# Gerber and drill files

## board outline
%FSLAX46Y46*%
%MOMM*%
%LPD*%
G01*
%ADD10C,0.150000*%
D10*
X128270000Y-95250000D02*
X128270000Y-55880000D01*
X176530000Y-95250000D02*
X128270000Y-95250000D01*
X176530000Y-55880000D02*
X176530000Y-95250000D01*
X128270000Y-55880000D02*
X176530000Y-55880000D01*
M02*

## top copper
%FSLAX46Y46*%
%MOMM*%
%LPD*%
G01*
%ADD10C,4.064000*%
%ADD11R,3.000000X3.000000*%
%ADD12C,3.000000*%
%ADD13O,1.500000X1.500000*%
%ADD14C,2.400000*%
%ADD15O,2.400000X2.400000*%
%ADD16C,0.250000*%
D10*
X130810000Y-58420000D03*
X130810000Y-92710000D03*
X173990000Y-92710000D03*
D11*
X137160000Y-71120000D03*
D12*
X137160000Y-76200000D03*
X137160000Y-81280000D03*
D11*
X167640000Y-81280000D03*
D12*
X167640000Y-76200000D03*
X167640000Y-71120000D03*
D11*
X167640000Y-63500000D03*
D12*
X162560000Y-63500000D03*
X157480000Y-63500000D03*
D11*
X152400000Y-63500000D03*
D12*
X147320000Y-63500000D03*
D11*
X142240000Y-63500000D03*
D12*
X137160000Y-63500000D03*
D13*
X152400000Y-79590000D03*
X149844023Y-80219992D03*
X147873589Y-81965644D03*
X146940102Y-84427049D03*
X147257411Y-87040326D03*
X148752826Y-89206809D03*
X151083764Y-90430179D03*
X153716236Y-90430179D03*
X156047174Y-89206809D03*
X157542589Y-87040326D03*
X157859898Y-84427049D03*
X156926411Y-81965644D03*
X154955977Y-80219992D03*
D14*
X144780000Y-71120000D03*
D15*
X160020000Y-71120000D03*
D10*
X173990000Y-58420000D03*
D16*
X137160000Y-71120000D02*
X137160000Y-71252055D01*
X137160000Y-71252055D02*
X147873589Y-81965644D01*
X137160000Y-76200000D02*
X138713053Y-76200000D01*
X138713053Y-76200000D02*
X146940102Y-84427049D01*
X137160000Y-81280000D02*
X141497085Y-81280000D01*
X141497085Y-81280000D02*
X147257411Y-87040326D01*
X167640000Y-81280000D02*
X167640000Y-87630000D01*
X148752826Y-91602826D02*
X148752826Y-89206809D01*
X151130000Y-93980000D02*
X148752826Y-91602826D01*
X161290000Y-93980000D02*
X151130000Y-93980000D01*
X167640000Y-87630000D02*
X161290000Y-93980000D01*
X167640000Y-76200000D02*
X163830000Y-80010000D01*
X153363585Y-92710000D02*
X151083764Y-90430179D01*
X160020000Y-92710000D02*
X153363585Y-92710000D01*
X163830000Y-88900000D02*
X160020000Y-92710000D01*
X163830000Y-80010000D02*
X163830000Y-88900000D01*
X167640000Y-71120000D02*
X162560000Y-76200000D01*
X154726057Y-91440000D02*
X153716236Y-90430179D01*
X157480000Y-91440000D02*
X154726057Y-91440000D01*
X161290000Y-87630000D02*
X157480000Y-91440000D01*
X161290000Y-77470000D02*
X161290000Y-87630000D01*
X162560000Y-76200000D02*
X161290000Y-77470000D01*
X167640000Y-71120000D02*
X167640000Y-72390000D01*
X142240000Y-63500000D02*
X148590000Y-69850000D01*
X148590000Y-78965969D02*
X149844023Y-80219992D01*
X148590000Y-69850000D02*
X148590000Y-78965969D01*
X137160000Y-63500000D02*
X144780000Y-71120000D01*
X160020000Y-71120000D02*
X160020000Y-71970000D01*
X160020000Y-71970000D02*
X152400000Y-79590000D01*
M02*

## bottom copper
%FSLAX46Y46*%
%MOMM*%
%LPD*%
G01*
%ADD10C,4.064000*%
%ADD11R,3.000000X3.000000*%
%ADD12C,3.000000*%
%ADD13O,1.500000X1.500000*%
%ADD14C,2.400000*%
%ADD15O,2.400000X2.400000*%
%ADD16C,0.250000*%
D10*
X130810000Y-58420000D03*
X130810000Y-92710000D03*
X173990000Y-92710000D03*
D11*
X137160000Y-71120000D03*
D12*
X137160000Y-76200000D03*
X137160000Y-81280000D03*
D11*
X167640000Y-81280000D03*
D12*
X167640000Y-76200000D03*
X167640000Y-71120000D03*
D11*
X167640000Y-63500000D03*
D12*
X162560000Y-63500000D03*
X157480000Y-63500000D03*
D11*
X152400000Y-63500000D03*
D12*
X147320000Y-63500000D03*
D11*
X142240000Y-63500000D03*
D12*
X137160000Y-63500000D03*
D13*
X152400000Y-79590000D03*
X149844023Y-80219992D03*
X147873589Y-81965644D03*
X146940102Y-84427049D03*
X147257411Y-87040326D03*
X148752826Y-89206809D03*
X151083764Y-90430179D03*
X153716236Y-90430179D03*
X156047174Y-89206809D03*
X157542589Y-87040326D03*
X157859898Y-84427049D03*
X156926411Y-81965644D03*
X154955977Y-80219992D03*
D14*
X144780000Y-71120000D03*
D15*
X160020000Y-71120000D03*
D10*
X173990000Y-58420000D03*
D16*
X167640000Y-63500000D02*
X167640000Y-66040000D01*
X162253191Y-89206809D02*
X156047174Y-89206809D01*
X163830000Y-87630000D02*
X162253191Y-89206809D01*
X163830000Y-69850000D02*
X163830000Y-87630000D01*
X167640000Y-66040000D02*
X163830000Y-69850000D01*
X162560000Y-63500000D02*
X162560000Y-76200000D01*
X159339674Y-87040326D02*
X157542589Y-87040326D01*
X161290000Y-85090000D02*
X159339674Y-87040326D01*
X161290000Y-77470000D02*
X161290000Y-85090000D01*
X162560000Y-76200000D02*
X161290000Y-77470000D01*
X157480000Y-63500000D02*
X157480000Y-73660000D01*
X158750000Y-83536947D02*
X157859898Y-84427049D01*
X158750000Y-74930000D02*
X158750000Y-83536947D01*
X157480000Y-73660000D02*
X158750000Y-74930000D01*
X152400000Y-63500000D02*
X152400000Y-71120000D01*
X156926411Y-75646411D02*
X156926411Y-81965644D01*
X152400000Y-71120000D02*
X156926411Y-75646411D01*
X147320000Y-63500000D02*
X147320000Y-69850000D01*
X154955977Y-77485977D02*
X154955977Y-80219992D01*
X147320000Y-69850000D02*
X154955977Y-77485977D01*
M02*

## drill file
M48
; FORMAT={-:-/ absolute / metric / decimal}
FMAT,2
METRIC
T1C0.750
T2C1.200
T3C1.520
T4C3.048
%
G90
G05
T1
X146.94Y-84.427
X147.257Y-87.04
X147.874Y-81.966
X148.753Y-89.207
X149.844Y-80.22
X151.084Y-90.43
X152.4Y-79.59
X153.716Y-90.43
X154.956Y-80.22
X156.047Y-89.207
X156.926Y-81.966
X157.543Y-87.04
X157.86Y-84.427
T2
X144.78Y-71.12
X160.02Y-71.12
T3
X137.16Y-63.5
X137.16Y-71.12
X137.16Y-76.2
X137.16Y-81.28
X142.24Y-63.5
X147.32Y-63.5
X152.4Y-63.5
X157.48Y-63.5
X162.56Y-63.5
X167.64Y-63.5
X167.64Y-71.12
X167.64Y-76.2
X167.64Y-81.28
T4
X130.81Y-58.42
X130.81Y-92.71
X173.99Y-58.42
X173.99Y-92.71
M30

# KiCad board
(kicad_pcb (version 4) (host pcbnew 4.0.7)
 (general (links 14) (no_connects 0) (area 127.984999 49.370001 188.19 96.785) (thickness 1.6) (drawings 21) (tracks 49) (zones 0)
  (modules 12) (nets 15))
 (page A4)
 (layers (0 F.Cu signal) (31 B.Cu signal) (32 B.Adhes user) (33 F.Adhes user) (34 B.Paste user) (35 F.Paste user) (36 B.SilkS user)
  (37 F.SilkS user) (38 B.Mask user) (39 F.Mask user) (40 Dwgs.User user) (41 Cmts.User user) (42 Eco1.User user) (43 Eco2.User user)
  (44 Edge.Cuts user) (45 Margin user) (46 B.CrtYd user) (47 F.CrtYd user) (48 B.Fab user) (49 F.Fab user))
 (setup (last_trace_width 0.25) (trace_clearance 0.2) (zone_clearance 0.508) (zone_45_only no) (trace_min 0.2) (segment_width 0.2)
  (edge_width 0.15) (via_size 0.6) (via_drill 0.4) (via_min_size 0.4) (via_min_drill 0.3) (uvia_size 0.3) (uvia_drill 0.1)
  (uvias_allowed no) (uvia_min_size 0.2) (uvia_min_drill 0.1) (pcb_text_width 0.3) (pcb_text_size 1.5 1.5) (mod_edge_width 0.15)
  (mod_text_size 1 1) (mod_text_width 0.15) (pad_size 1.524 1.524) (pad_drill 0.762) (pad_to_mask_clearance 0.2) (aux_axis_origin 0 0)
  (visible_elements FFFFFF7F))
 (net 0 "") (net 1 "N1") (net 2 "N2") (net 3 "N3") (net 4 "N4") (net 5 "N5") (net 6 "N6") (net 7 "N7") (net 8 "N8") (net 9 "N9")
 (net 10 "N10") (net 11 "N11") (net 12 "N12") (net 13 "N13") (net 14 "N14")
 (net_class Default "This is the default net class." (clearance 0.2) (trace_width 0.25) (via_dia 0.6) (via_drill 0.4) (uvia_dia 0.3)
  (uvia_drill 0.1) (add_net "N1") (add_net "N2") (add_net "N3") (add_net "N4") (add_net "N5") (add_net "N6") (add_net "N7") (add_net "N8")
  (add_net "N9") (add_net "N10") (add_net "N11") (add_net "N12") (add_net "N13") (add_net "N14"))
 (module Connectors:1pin (layer F.Cu) (at 130.81 58.42)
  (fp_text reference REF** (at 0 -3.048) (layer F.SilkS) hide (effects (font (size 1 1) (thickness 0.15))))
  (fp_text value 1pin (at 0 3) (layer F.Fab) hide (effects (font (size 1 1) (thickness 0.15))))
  (pad 1 thru_hole circle (at 0 0) (size 4.064 4.064) (drill 3.048) (layers *.Cu *.Mask)))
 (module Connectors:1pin (layer F.Cu) (at 130.81 92.71)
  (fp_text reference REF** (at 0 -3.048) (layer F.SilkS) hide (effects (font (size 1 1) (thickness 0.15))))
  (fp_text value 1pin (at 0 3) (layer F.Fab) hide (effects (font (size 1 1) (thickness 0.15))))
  (pad 1 thru_hole circle (at 0 0) (size 4.064 4.064) (drill 3.048) (layers *.Cu *.Mask)))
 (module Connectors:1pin (layer F.Cu) (at 173.99 92.71)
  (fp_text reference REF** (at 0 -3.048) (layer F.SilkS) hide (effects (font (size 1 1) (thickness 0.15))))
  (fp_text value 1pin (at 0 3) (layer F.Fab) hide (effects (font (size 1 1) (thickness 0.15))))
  (pad 1 thru_hole circle (at 0 0) (size 4.064 4.064) (drill 3.048) (layers *.Cu *.Mask)))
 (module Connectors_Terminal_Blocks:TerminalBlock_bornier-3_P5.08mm (layer F.Cu) (at 137.16 71.12 270)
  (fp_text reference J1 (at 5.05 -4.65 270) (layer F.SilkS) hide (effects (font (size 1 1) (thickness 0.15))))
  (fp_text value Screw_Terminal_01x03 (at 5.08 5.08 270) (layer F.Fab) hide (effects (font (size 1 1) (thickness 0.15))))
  (pad 1 thru_hole rect (at 0 0 270) (size 3 3) (drill 1.52) (layers *.Cu *.Mask) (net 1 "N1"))
  (pad 2 thru_hole circle (at 5.08 0 270) (size 3 3) (drill 1.52) (layers *.Cu *.Mask) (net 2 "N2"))
  (pad 3 thru_hole circle (at 10.16 0 270) (size 3 3) (drill 1.52) (layers *.Cu *.Mask) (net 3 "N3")))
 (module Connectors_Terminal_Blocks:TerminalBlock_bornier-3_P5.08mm (layer F.Cu) (at 167.64 81.28 90)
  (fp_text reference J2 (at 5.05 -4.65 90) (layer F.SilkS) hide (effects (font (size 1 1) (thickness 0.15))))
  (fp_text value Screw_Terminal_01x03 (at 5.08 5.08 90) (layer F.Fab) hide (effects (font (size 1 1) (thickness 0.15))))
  (pad 1 thru_hole rect (at 0 0 90) (size 3 3) (drill 1.52) (layers *.Cu *.Mask) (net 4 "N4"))
  (pad 2 thru_hole circle (at 5.08 0 90) (size 3 3) (drill 1.52) (layers *.Cu *.Mask) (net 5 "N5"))
  (pad 3 thru_hole circle (at 10.16 0 90) (size 3 3) (drill 1.52) (layers *.Cu *.Mask) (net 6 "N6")))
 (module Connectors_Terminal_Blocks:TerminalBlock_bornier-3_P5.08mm (layer F.Cu) (at 167.64 63.5 180)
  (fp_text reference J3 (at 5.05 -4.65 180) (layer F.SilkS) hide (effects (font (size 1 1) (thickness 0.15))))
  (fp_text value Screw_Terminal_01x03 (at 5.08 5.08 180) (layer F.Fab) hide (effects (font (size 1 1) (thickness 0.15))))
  (pad 1 thru_hole rect (at 0 0 180) (size 3 3) (drill 1.52) (layers *.Cu *.Mask) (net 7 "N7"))
  (pad 2 thru_hole circle (at 5.08 0 180) (size 3 3) (drill 1.52) (layers *.Cu *.Mask) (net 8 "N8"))
  (pad 3 thru_hole circle (at 10.16 0 180) (size 3 3) (drill 1.52) (layers *.Cu *.Mask) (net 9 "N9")))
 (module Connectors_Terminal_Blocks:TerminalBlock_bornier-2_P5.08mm (layer F.Cu) (at 152.4 63.5 180)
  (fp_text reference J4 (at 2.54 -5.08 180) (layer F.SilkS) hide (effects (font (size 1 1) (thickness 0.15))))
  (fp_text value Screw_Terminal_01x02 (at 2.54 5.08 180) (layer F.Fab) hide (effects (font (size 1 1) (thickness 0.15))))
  (pad 1 thru_hole rect (at 0 0 180) (size 3 3) (drill 1.52) (layers *.Cu *.Mask) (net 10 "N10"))
  (pad 2 thru_hole circle (at 5.08 0 180) (size 3 3) (drill 1.52) (layers *.Cu *.Mask) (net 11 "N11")))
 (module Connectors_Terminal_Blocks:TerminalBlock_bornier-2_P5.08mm (layer F.Cu) (at 142.24 63.5 180)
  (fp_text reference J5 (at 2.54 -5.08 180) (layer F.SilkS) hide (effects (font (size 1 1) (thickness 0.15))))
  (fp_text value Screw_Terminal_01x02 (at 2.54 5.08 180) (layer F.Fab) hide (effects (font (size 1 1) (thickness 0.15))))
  (pad 1 thru_hole rect (at 0 0 180) (size 3 3) (drill 1.52) (layers *.Cu *.Mask) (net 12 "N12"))
  (pad 2 thru_hole circle (at 5.08 0 180) (size 3 3) (drill 1.52) (layers *.Cu *.Mask) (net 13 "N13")))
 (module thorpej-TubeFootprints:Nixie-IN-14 (layer F.Cu) (at 152.4 85.09)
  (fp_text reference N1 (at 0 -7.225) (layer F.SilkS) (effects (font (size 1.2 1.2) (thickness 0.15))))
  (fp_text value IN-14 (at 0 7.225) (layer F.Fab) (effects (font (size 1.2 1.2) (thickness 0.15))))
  (pad 1 thru_hole oval (at 0 -5.5) (size 1.5 1.5) (drill 0.75) (layers *.Cu *.Mask) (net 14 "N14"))
  (pad 2 thru_hole oval (at -2.555977 -4.870008) (size 1.5 1.5) (drill 0.75) (layers *.Cu *.Mask) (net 12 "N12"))
  (pad 3 thru_hole oval (at -4.526411 -3.124356) (size 1.5 1.5) (drill 0.75) (layers *.Cu *.Mask) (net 1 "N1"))
  (pad 4 thru_hole oval (at -5.459898 -0.662951) (size 1.5 1.5) (drill 0.75) (layers *.Cu *.Mask) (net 2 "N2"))
  (pad 5 thru_hole oval (at -5.142589 1.950326) (size 1.5 1.5) (drill 0.75) (layers *.Cu *.Mask) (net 3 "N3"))
  (pad 6 thru_hole oval (at -3.647174 4.116809) (size 1.5 1.5) (drill 0.75) (layers *.Cu *.Mask) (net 4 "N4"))
  (pad 7 thru_hole oval (at -1.316236 5.340179) (size 1.5 1.5) (drill 0.75) (layers *.Cu *.Mask) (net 5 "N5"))
  (pad 8 thru_hole oval (at 1.316236 5.340179) (size 1.5 1.5) (drill 0.75) (layers *.Cu *.Mask) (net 6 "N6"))
  (pad 9 thru_hole oval (at 3.647174 4.116809) (size 1.5 1.5) (drill 0.75) (layers *.Cu *.Mask) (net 7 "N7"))
  (pad 10 thru_hole oval (at 5.142589 1.950326) (size 1.5 1.5) (drill 0.75) (layers *.Cu *.Mask) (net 8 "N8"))
  (pad 11 thru_hole oval (at 5.459898 -0.662951) (size 1.5 1.5) (drill 0.75) (layers *.Cu *.Mask) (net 9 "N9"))
  (pad 12 thru_hole oval (at 4.526411 -3.124356) (size 1.5 1.5) (drill 0.75) (layers *.Cu *.Mask) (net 10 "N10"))
  (pad 13 thru_hole oval (at 2.555977 -4.870008) (size 1.5 1.5) (drill 0.75) (layers *.Cu *.Mask) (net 11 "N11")))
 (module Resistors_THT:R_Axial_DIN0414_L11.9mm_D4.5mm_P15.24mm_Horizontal (layer F.Cu) (at 144.78 71.12)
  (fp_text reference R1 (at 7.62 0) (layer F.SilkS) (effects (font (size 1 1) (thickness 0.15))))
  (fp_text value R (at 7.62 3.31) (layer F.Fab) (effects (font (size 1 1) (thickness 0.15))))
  (pad 1 thru_hole circle (at 0 0) (size 2.4 2.4) (drill 1.2) (layers *.Cu *.Mask) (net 13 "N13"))
  (pad 2 thru_hole oval (at 15.24 0) (size 2.4 2.4) (drill 1.2) (layers *.Cu *.Mask) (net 14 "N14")))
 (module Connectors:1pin (layer F.Cu) (at 173.99 58.42)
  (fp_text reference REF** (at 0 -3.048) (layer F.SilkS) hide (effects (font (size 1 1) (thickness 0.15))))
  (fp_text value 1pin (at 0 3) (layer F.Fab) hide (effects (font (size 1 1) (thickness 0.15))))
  (pad 1 thru_hole circle (at 0 0) (size 4.064 4.064) (drill 3.048) (layers *.Cu *.Mask)))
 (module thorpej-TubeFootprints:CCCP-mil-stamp (layer F.Cu) (at 167.64 88.9)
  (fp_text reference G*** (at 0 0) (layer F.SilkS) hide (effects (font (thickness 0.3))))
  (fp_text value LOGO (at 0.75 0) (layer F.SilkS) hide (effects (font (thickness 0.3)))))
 (gr_line (start 128.27 95.25) (end 128.27 55.88) (angle 90) (layer Edge.Cuts) (width 0.15))
 (gr_line (start 176.53 95.25) (end 128.27 95.25) (angle 90) (layer Edge.Cuts) (width 0.15))
 (gr_line (start 176.53 55.88) (end 176.53 95.25) (angle 90) (layer Edge.Cuts) (width 0.15))
 (gr_line (start 128.27 55.88) (end 176.53 55.88) (angle 90) (layer Edge.Cuts) (width 0.15))
 (segment (start 137.16 71.12) (end 137.16 71.252055) (width 0.25) (layer F.Cu) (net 1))
 (segment (start 137.16 71.252055) (end 147.873589 81.965644) (width 0.25) (layer F.Cu) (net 1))
 (segment (start 137.16 76.2) (end 138.713053 76.2) (width 0.25) (layer F.Cu) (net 2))
 (segment (start 138.713053 76.2) (end 146.940102 84.427049) (width 0.25) (layer F.Cu) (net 2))
 (segment (start 137.16 81.28) (end 141.497085 81.28) (width 0.25) (layer F.Cu) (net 3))
 (segment (start 141.497085 81.28) (end 147.257411 87.040326) (width 0.25) (layer F.Cu) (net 3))
 (segment (start 167.64 81.28) (end 167.64 87.63) (width 0.25) (layer F.Cu) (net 4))
 (segment (start 148.752826 91.602826) (end 148.752826 89.206809) (width 0.25) (layer F.Cu) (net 4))
 (segment (start 151.13 93.98) (end 148.752826 91.602826) (width 0.25) (layer F.Cu) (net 4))
 (segment (start 161.29 93.98) (end 151.13 93.98) (width 0.25) (layer F.Cu) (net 4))
 (segment (start 167.64 87.63) (end 161.29 93.98) (width 0.25) (layer F.Cu) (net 4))
 (segment (start 167.64 76.2) (end 163.83 80.01) (width 0.25) (layer F.Cu) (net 5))
 (segment (start 153.363585 92.71) (end 151.083764 90.430179) (width 0.25) (layer F.Cu) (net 5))
 (segment (start 160.02 92.71) (end 153.363585 92.71) (width 0.25) (layer F.Cu) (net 5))
 (segment (start 163.83 88.9) (end 160.02 92.71) (width 0.25) (layer F.Cu) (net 5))
 (segment (start 163.83 80.01) (end 163.83 88.9) (width 0.25) (layer F.Cu) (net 5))
 (segment (start 167.64 71.12) (end 162.56 76.2) (width 0.25) (layer F.Cu) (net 6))
 (segment (start 154.726057 91.44) (end 153.716236 90.430179) (width 0.25) (layer F.Cu) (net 6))
 (segment (start 157.48 91.44) (end 154.726057 91.44) (width 0.25) (layer F.Cu) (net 6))
 (segment (start 161.29 87.63) (end 157.48 91.44) (width 0.25) (layer F.Cu) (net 6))
 (segment (start 161.29 77.47) (end 161.29 87.63) (width 0.25) (layer F.Cu) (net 6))
 (segment (start 162.56 76.2) (end 161.29 77.47) (width 0.25) (layer F.Cu) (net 6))
 (segment (start 167.64 71.12) (end 167.64 72.39) (width 0.25) (layer F.Cu) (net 6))
 (segment (start 167.64 63.5) (end 167.64 66.04) (width 0.25) (layer B.Cu) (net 7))
 (segment (start 162.253191 89.206809) (end 156.047174 89.206809) (width 0.25) (layer B.Cu) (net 7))
 (segment (start 163.83 87.63) (end 162.253191 89.206809) (width 0.25) (layer B.Cu) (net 7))
 (segment (start 163.83 69.85) (end 163.83 87.63) (width 0.25) (layer B.Cu) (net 7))
 (segment (start 167.64 66.04) (end 163.83 69.85) (width 0.25) (layer B.Cu) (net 7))
 (segment (start 162.56 63.5) (end 162.56 76.2) (width 0.25) (layer B.Cu) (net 8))
 (segment (start 159.339674 87.040326) (end 157.542589 87.040326) (width 0.25) (layer B.Cu) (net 8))
 (segment (start 161.29 85.09) (end 159.339674 87.040326) (width 0.25) (layer B.Cu) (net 8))
 (segment (start 161.29 77.47) (end 161.29 85.09) (width 0.25) (layer B.Cu) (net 8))
 (segment (start 162.56 76.2) (end 161.29 77.47) (width 0.25) (layer B.Cu) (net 8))
 (segment (start 157.48 63.5) (end 157.48 73.66) (width 0.25) (layer B.Cu) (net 9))
 (segment (start 158.75 83.536947) (end 157.859898 84.427049) (width 0.25) (layer B.Cu) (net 9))
 (segment (start 158.75 74.93) (end 158.75 83.536947) (width 0.25) (layer B.Cu) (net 9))
 (segment (start 157.48 73.66) (end 158.75 74.93) (width 0.25) (layer B.Cu) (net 9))
 (segment (start 152.4 63.5) (end 152.4 71.12) (width 0.25) (layer B.Cu) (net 10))
 (segment (start 156.926411 75.646411) (end 156.926411 81.965644) (width 0.25) (layer B.Cu) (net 10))
 (segment (start 152.4 71.12) (end 156.926411 75.646411) (width 0.25) (layer B.Cu) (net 10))
 (segment (start 147.32 63.5) (end 147.32 69.85) (width 0.25) (layer B.Cu) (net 11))
 (segment (start 154.955977 77.485977) (end 154.955977 80.219992) (width 0.25) (layer B.Cu) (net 11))
 (segment (start 147.32 69.85) (end 154.955977 77.485977) (width 0.25) (layer B.Cu) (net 11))
 (segment (start 142.24 63.5) (end 148.59 69.85) (width 0.25) (layer F.Cu) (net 12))
 (segment (start 148.59 78.965969) (end 149.844023 80.219992) (width 0.25) (layer F.Cu) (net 12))
 (segment (start 148.59 69.85) (end 148.59 78.965969) (width 0.25) (layer F.Cu) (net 12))
 (segment (start 137.16 63.5) (end 144.78 71.12) (width 0.25) (layer F.Cu) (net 13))
 (segment (start 160.02 71.12) (end 160.02 71.97) (width 0.25) (layer F.Cu) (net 14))
 (segment (start 160.02 71.97) (end 152.4 79.59) (width 0.25) (layer F.Cu) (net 14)))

